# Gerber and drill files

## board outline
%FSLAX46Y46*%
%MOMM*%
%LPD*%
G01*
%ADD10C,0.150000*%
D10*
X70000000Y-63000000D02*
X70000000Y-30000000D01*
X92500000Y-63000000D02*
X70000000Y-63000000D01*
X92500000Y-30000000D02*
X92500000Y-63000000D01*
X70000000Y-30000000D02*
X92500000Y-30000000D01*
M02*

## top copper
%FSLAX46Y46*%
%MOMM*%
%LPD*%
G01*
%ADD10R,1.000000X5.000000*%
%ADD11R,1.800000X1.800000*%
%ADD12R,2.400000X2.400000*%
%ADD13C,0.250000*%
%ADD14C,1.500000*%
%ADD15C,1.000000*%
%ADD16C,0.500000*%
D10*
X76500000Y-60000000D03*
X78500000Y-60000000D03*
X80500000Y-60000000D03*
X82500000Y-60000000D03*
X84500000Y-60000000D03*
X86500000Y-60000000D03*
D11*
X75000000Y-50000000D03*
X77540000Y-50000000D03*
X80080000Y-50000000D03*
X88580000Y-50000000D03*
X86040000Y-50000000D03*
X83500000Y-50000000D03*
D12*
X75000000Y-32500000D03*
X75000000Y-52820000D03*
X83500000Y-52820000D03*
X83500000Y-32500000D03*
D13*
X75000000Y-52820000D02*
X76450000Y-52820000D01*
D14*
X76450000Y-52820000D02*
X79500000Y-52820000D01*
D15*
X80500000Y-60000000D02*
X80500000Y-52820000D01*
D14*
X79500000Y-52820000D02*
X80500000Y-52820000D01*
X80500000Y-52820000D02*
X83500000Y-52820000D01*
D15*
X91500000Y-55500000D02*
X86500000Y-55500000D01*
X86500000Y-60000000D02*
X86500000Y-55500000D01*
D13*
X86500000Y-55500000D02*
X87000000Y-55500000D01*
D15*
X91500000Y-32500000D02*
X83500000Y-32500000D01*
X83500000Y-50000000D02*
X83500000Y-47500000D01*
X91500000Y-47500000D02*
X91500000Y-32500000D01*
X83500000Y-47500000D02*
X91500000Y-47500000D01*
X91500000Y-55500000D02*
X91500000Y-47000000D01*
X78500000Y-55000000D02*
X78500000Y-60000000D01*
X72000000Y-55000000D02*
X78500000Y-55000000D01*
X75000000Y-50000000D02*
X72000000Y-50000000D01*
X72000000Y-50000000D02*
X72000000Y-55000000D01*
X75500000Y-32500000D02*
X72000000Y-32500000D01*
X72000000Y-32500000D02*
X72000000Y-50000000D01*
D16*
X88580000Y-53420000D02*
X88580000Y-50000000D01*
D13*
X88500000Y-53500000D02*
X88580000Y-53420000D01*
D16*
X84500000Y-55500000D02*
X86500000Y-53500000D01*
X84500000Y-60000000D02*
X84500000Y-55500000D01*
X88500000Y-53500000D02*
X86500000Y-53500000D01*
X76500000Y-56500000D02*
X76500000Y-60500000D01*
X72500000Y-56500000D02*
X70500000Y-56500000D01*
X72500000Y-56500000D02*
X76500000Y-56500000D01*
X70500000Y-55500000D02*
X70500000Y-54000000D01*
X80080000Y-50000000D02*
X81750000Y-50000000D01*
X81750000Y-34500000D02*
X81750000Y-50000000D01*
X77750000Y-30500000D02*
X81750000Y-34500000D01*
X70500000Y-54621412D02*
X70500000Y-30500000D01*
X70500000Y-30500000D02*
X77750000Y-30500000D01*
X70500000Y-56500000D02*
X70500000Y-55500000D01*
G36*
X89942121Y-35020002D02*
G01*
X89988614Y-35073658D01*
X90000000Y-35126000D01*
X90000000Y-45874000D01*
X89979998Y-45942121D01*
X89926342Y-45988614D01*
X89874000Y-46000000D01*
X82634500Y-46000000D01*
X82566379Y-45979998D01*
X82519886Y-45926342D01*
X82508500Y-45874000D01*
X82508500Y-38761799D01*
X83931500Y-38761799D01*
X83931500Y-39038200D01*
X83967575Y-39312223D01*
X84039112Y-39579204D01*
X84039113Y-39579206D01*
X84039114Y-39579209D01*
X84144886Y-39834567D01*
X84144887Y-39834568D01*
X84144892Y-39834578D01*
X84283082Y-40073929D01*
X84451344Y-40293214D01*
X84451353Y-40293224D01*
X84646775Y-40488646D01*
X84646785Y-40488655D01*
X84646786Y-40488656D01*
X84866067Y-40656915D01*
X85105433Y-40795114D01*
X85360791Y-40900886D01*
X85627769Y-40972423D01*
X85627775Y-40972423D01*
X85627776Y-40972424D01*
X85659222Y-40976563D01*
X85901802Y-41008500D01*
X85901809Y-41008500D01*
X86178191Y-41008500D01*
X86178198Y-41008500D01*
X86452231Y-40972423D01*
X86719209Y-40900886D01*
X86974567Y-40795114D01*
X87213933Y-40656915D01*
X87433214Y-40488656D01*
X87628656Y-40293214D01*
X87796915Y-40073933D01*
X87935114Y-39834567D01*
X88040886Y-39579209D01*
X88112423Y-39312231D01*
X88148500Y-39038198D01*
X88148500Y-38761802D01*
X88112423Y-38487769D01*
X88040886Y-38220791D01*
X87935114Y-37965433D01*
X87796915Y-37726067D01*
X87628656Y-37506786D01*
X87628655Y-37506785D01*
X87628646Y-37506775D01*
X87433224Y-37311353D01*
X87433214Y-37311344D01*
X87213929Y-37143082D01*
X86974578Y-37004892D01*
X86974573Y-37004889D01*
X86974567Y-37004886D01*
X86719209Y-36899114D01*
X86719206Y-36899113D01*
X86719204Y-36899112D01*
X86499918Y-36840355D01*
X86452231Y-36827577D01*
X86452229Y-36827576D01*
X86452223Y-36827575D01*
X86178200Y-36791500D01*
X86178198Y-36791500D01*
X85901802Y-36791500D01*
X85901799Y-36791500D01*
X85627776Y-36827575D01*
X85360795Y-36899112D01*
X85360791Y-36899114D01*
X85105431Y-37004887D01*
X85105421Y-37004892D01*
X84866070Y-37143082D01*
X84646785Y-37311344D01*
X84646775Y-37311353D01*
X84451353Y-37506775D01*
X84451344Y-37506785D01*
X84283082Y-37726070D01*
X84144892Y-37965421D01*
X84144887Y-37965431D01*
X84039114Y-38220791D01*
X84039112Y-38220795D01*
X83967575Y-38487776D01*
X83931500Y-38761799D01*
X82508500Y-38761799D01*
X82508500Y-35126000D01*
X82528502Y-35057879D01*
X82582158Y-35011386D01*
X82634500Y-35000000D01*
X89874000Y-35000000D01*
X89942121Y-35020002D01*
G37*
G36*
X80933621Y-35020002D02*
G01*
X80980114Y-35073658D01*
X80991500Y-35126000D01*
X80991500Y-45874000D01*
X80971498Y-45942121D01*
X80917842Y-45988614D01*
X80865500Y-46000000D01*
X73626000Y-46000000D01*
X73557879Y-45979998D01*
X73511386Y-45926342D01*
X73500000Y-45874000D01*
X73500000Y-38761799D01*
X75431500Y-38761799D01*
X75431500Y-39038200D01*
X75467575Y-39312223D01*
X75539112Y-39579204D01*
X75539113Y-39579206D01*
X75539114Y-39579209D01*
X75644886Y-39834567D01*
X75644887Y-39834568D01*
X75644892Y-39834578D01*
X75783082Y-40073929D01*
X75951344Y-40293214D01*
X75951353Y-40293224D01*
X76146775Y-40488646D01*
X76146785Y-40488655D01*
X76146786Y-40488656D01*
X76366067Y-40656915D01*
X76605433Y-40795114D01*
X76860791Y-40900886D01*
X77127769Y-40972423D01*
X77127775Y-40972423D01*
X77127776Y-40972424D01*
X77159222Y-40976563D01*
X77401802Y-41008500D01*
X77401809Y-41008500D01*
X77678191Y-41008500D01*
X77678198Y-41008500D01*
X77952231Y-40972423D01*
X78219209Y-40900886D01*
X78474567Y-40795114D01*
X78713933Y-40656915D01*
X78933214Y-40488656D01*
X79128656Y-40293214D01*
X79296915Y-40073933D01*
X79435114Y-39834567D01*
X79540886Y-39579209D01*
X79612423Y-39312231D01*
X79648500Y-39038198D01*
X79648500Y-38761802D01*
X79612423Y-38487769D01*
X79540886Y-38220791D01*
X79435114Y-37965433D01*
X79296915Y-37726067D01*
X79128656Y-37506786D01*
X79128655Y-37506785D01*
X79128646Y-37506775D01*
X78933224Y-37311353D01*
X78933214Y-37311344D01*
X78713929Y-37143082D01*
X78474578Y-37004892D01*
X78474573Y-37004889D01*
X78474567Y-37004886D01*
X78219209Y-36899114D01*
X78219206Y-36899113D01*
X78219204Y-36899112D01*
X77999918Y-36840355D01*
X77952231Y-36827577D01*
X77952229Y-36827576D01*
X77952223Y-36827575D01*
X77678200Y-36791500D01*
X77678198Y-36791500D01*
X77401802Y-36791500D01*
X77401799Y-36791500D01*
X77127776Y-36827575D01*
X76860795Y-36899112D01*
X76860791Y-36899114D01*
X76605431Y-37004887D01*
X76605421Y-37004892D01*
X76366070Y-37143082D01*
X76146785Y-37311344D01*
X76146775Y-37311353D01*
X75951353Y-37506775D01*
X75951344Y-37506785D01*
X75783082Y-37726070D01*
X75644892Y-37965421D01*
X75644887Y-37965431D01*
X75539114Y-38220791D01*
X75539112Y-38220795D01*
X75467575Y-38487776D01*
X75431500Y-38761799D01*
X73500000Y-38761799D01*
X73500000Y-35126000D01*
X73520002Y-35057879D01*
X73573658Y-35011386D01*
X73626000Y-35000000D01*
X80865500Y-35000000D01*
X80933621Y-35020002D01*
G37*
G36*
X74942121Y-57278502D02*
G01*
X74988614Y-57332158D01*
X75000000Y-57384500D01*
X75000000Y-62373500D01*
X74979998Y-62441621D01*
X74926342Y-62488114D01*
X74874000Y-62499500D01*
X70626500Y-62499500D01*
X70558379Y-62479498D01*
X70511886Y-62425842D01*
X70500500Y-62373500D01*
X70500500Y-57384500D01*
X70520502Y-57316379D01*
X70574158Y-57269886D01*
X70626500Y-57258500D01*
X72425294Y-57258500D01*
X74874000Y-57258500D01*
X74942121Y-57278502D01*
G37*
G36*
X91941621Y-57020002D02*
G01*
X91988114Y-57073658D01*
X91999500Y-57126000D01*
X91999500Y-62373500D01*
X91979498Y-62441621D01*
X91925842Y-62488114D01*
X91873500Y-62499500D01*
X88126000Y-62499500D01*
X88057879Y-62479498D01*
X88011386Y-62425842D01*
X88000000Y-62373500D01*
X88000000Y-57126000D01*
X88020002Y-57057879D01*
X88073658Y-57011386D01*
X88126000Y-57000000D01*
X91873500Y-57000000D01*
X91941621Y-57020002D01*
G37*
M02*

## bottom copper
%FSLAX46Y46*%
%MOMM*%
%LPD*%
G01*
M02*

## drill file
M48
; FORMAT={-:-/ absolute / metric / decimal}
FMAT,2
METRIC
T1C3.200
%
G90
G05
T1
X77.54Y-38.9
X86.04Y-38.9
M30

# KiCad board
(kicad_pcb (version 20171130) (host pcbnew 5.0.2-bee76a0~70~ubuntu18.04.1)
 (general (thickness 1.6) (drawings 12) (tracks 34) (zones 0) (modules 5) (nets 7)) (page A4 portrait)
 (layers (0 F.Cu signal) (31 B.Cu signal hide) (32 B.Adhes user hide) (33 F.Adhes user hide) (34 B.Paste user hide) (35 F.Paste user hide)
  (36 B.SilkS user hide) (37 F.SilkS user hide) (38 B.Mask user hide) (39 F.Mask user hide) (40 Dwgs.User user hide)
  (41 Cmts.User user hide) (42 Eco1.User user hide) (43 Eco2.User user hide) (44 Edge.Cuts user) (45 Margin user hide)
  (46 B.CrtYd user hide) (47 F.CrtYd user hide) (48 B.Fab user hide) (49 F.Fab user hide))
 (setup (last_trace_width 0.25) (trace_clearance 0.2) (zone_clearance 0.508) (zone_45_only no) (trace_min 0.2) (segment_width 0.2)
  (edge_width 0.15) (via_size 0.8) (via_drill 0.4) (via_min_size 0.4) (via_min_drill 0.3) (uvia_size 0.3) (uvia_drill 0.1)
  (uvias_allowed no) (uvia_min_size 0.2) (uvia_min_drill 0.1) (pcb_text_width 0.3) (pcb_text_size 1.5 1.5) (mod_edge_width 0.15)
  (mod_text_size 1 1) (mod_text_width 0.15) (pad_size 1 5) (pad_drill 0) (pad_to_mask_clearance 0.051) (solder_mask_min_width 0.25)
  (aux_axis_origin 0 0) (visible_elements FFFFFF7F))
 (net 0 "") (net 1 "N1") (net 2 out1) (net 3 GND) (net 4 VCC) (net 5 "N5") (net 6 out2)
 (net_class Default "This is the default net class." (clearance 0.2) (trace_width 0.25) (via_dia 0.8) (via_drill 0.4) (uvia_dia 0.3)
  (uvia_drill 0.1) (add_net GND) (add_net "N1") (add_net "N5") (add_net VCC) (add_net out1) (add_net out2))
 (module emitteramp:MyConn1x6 (layer F.Cu) (at 81.5 60)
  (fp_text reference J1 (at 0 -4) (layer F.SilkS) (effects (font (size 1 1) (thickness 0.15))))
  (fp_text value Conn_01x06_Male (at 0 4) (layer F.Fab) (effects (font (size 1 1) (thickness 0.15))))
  (pad 1 smd rect (at -5 0) (size 1 5) (layers F.Cu F.Paste F.Mask) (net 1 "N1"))
  (pad 2 smd rect (at -3 0) (size 1 5) (layers F.Cu F.Paste F.Mask) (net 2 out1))
  (pad 3 smd rect (at -1 0) (size 1 5) (layers F.Cu F.Paste F.Mask) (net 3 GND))
  (pad 4 smd rect (at 1 0) (size 1 5) (layers F.Cu F.Paste F.Mask) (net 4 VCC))
  (pad 5 smd rect (at 3 0) (size 1 5) (layers F.Cu F.Paste F.Mask) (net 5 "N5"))
  (pad 6 smd rect (at 5 0) (size 1 5) (layers F.Cu F.Paste F.Mask) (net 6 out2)))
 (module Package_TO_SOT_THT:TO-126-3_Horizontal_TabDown (layer F.Cu) (at 75 50)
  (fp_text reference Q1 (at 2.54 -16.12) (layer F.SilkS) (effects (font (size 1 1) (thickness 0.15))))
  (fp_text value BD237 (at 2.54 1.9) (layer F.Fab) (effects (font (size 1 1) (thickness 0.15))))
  (pad "" np_thru_hole oval (at 2.54 -11.1) (size 3.2 3.2) (drill 3.2) (layers *.Cu *.Mask))
  (pad 1 smd rect (at 0 0) (size 1.8 1.8) (layers F.Cu F.Paste F.Mask) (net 2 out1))
  (pad 2 smd rect (at 2.54 0) (size 1.8 1.8) (layers F.Cu F.Paste F.Mask) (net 4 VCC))
  (pad 3 smd rect (at 5.08 0) (size 1.8 1.8) (layers F.Cu F.Paste F.Mask) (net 1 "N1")))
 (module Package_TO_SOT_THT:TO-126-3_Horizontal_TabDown (layer F.Cu) (at 83.5 50)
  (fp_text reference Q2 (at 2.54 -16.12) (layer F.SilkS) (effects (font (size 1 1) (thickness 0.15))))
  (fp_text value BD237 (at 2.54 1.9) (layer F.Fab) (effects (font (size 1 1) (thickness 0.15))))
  (pad 3 smd rect (at 5.08 0) (size 1.8 1.8) (layers F.Cu F.Paste F.Mask) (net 5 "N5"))
  (pad 2 smd rect (at 2.54 0) (size 1.8 1.8) (layers F.Cu F.Paste F.Mask) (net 4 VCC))
  (pad 1 smd rect (at 0 0) (size 1.8 1.8) (layers F.Cu F.Paste F.Mask) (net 6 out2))
  (pad "" np_thru_hole oval (at 2.54 -11.1) (size 3.2 3.2) (drill 3.2) (layers *.Cu *.Mask)))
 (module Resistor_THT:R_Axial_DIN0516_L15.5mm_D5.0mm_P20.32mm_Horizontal (layer F.Cu) (at 75 32.5 270)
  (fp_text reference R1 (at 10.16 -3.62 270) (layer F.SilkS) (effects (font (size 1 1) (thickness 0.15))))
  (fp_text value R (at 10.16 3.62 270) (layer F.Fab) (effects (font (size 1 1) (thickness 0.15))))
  (pad 1 smd rect (at 0 0 270) (size 2.4 2.4) (layers F.Cu F.Paste F.Mask) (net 2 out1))
  (pad 2 smd rect (at 20.32 0 270) (size 2.4 2.4) (layers F.Cu F.Paste F.Mask) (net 3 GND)))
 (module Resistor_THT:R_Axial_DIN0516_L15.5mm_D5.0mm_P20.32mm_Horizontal (layer F.Cu) (at 83.5 32.5 270)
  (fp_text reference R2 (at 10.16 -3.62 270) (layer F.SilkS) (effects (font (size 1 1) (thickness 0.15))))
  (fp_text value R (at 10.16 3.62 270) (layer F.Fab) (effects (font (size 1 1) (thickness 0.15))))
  (pad 2 smd rect (at 20.32 0 270) (size 2.4 2.4) (layers F.Cu F.Paste F.Mask) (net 3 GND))
  (pad 1 smd rect (at 0 0 270) (size 2.4 2.4) (layers F.Cu F.Paste F.Mask) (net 6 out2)))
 (gr_line (start 70 63) (end 70 30) (layer Edge.Cuts) (width 0.15))
 (gr_line (start 92.5 63) (end 70 63) (layer Edge.Cuts) (width 0.15))
 (gr_line (start 92.5 30) (end 92.5 63) (layer Edge.Cuts) (width 0.15))
 (gr_line (start 70 30) (end 92.5 30) (layer Edge.Cuts) (width 0.15))
 (segment (start 75 52.82) (end 76.45 52.82) (width 0.25) (layer F.Cu) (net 3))
 (segment (start 76.45 52.82) (end 79.5 52.82) (width 1.5) (layer F.Cu) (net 3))
 (segment (start 80.5 60) (end 80.5 52.82) (width 1) (layer F.Cu) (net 3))
 (segment (start 79.5 52.82) (end 80.5 52.82) (width 1.5) (layer F.Cu) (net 3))
 (segment (start 80.5 52.82) (end 83.5 52.82) (width 1.5) (layer F.Cu) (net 3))
 (segment (start 91.5 55.5) (end 86.5 55.5) (width 1) (layer F.Cu) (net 6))
 (segment (start 86.5 60) (end 86.5 55.5) (width 1) (layer F.Cu) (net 6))
 (segment (start 86.5 55.5) (end 87 55.5) (width 0.25) (layer F.Cu) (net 6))
 (segment (start 91.5 32.5) (end 83.5 32.5) (width 1) (layer F.Cu) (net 6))
 (segment (start 83.5 50) (end 83.5 47.5) (width 1) (layer F.Cu) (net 6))
 (segment (start 91.5 47.5) (end 91.5 32.5) (width 1) (layer F.Cu) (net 6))
 (segment (start 83.5 47.5) (end 91.5 47.5) (width 1) (layer F.Cu) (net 6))
 (segment (start 91.5 55.5) (end 91.5 47) (width 1) (layer F.Cu) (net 6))
 (segment (start 78.5 55) (end 78.5 60) (width 1) (layer F.Cu) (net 2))
 (segment (start 72 55) (end 78.5 55) (width 1) (layer F.Cu) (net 2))
 (segment (start 75 50) (end 72 50) (width 1) (layer F.Cu) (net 2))
 (segment (start 72 50) (end 72 55) (width 1) (layer F.Cu) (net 2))
 (segment (start 75.5 32.5) (end 72 32.5) (width 1) (layer F.Cu) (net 2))
 (segment (start 72 32.5) (end 72 50) (width 1) (layer F.Cu) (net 2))
 (segment (start 88.58 53.42) (end 88.58 50) (width 0.5) (layer F.Cu) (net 5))
 (segment (start 88.5 53.5) (end 88.58 53.42) (width 0.25) (layer F.Cu) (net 5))
 (segment (start 84.5 55.5) (end 86.5 53.5) (width 0.5) (layer F.Cu) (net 5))
 (segment (start 84.5 60) (end 84.5 55.5) (width 0.5) (layer F.Cu) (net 5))
 (segment (start 88.5 53.5) (end 86.5 53.5) (width 0.5) (layer F.Cu) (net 5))
 (segment (start 76.5 56.5) (end 76.5 60.5) (width 0.5) (layer F.Cu) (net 1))
 (segment (start 72.5 56.5) (end 70.5 56.5) (width 0.5) (layer F.Cu) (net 1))
 (segment (start 72.5 56.5) (end 76.5 56.5) (width 0.5) (layer F.Cu) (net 1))
 (segment (start 70.5 55.5) (end 70.5 54) (width 0.5) (layer F.Cu) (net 1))
 (segment (start 80.08 50) (end 81.75 50) (width 0.5) (layer F.Cu) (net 1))
 (segment (start 81.75 34.5) (end 81.75 50) (width 0.5) (layer F.Cu) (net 1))
 (segment (start 77.75 30.5) (end 81.75 34.5) (width 0.5) (layer F.Cu) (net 1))
 (segment (start 70.5 54.621412) (end 70.5 30.5) (width 0.5) (layer F.Cu) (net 1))
 (segment (start 70.5 30.5) (end 77.75 30.5) (width 0.5) (layer F.Cu) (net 1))
 (segment (start 70.5 56.5) (end 70.5 55.5) (width 0.5) (layer F.Cu) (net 1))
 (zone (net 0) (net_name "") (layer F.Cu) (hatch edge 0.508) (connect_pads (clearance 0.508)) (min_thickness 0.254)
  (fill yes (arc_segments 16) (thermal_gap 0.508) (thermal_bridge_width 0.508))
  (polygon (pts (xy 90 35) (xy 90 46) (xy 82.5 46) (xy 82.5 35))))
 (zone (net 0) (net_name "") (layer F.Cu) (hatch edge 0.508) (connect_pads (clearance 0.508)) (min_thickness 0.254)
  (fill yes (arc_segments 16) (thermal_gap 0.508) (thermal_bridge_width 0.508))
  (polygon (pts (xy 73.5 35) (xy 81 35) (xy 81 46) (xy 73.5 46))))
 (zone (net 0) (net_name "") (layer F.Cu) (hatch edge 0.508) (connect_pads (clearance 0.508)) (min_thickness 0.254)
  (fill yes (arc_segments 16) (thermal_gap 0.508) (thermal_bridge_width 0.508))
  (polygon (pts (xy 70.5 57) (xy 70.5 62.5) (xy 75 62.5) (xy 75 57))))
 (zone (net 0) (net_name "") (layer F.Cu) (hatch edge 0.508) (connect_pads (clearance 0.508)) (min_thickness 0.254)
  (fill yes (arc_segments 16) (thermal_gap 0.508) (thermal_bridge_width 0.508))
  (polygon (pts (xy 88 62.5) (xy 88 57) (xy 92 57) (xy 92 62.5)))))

